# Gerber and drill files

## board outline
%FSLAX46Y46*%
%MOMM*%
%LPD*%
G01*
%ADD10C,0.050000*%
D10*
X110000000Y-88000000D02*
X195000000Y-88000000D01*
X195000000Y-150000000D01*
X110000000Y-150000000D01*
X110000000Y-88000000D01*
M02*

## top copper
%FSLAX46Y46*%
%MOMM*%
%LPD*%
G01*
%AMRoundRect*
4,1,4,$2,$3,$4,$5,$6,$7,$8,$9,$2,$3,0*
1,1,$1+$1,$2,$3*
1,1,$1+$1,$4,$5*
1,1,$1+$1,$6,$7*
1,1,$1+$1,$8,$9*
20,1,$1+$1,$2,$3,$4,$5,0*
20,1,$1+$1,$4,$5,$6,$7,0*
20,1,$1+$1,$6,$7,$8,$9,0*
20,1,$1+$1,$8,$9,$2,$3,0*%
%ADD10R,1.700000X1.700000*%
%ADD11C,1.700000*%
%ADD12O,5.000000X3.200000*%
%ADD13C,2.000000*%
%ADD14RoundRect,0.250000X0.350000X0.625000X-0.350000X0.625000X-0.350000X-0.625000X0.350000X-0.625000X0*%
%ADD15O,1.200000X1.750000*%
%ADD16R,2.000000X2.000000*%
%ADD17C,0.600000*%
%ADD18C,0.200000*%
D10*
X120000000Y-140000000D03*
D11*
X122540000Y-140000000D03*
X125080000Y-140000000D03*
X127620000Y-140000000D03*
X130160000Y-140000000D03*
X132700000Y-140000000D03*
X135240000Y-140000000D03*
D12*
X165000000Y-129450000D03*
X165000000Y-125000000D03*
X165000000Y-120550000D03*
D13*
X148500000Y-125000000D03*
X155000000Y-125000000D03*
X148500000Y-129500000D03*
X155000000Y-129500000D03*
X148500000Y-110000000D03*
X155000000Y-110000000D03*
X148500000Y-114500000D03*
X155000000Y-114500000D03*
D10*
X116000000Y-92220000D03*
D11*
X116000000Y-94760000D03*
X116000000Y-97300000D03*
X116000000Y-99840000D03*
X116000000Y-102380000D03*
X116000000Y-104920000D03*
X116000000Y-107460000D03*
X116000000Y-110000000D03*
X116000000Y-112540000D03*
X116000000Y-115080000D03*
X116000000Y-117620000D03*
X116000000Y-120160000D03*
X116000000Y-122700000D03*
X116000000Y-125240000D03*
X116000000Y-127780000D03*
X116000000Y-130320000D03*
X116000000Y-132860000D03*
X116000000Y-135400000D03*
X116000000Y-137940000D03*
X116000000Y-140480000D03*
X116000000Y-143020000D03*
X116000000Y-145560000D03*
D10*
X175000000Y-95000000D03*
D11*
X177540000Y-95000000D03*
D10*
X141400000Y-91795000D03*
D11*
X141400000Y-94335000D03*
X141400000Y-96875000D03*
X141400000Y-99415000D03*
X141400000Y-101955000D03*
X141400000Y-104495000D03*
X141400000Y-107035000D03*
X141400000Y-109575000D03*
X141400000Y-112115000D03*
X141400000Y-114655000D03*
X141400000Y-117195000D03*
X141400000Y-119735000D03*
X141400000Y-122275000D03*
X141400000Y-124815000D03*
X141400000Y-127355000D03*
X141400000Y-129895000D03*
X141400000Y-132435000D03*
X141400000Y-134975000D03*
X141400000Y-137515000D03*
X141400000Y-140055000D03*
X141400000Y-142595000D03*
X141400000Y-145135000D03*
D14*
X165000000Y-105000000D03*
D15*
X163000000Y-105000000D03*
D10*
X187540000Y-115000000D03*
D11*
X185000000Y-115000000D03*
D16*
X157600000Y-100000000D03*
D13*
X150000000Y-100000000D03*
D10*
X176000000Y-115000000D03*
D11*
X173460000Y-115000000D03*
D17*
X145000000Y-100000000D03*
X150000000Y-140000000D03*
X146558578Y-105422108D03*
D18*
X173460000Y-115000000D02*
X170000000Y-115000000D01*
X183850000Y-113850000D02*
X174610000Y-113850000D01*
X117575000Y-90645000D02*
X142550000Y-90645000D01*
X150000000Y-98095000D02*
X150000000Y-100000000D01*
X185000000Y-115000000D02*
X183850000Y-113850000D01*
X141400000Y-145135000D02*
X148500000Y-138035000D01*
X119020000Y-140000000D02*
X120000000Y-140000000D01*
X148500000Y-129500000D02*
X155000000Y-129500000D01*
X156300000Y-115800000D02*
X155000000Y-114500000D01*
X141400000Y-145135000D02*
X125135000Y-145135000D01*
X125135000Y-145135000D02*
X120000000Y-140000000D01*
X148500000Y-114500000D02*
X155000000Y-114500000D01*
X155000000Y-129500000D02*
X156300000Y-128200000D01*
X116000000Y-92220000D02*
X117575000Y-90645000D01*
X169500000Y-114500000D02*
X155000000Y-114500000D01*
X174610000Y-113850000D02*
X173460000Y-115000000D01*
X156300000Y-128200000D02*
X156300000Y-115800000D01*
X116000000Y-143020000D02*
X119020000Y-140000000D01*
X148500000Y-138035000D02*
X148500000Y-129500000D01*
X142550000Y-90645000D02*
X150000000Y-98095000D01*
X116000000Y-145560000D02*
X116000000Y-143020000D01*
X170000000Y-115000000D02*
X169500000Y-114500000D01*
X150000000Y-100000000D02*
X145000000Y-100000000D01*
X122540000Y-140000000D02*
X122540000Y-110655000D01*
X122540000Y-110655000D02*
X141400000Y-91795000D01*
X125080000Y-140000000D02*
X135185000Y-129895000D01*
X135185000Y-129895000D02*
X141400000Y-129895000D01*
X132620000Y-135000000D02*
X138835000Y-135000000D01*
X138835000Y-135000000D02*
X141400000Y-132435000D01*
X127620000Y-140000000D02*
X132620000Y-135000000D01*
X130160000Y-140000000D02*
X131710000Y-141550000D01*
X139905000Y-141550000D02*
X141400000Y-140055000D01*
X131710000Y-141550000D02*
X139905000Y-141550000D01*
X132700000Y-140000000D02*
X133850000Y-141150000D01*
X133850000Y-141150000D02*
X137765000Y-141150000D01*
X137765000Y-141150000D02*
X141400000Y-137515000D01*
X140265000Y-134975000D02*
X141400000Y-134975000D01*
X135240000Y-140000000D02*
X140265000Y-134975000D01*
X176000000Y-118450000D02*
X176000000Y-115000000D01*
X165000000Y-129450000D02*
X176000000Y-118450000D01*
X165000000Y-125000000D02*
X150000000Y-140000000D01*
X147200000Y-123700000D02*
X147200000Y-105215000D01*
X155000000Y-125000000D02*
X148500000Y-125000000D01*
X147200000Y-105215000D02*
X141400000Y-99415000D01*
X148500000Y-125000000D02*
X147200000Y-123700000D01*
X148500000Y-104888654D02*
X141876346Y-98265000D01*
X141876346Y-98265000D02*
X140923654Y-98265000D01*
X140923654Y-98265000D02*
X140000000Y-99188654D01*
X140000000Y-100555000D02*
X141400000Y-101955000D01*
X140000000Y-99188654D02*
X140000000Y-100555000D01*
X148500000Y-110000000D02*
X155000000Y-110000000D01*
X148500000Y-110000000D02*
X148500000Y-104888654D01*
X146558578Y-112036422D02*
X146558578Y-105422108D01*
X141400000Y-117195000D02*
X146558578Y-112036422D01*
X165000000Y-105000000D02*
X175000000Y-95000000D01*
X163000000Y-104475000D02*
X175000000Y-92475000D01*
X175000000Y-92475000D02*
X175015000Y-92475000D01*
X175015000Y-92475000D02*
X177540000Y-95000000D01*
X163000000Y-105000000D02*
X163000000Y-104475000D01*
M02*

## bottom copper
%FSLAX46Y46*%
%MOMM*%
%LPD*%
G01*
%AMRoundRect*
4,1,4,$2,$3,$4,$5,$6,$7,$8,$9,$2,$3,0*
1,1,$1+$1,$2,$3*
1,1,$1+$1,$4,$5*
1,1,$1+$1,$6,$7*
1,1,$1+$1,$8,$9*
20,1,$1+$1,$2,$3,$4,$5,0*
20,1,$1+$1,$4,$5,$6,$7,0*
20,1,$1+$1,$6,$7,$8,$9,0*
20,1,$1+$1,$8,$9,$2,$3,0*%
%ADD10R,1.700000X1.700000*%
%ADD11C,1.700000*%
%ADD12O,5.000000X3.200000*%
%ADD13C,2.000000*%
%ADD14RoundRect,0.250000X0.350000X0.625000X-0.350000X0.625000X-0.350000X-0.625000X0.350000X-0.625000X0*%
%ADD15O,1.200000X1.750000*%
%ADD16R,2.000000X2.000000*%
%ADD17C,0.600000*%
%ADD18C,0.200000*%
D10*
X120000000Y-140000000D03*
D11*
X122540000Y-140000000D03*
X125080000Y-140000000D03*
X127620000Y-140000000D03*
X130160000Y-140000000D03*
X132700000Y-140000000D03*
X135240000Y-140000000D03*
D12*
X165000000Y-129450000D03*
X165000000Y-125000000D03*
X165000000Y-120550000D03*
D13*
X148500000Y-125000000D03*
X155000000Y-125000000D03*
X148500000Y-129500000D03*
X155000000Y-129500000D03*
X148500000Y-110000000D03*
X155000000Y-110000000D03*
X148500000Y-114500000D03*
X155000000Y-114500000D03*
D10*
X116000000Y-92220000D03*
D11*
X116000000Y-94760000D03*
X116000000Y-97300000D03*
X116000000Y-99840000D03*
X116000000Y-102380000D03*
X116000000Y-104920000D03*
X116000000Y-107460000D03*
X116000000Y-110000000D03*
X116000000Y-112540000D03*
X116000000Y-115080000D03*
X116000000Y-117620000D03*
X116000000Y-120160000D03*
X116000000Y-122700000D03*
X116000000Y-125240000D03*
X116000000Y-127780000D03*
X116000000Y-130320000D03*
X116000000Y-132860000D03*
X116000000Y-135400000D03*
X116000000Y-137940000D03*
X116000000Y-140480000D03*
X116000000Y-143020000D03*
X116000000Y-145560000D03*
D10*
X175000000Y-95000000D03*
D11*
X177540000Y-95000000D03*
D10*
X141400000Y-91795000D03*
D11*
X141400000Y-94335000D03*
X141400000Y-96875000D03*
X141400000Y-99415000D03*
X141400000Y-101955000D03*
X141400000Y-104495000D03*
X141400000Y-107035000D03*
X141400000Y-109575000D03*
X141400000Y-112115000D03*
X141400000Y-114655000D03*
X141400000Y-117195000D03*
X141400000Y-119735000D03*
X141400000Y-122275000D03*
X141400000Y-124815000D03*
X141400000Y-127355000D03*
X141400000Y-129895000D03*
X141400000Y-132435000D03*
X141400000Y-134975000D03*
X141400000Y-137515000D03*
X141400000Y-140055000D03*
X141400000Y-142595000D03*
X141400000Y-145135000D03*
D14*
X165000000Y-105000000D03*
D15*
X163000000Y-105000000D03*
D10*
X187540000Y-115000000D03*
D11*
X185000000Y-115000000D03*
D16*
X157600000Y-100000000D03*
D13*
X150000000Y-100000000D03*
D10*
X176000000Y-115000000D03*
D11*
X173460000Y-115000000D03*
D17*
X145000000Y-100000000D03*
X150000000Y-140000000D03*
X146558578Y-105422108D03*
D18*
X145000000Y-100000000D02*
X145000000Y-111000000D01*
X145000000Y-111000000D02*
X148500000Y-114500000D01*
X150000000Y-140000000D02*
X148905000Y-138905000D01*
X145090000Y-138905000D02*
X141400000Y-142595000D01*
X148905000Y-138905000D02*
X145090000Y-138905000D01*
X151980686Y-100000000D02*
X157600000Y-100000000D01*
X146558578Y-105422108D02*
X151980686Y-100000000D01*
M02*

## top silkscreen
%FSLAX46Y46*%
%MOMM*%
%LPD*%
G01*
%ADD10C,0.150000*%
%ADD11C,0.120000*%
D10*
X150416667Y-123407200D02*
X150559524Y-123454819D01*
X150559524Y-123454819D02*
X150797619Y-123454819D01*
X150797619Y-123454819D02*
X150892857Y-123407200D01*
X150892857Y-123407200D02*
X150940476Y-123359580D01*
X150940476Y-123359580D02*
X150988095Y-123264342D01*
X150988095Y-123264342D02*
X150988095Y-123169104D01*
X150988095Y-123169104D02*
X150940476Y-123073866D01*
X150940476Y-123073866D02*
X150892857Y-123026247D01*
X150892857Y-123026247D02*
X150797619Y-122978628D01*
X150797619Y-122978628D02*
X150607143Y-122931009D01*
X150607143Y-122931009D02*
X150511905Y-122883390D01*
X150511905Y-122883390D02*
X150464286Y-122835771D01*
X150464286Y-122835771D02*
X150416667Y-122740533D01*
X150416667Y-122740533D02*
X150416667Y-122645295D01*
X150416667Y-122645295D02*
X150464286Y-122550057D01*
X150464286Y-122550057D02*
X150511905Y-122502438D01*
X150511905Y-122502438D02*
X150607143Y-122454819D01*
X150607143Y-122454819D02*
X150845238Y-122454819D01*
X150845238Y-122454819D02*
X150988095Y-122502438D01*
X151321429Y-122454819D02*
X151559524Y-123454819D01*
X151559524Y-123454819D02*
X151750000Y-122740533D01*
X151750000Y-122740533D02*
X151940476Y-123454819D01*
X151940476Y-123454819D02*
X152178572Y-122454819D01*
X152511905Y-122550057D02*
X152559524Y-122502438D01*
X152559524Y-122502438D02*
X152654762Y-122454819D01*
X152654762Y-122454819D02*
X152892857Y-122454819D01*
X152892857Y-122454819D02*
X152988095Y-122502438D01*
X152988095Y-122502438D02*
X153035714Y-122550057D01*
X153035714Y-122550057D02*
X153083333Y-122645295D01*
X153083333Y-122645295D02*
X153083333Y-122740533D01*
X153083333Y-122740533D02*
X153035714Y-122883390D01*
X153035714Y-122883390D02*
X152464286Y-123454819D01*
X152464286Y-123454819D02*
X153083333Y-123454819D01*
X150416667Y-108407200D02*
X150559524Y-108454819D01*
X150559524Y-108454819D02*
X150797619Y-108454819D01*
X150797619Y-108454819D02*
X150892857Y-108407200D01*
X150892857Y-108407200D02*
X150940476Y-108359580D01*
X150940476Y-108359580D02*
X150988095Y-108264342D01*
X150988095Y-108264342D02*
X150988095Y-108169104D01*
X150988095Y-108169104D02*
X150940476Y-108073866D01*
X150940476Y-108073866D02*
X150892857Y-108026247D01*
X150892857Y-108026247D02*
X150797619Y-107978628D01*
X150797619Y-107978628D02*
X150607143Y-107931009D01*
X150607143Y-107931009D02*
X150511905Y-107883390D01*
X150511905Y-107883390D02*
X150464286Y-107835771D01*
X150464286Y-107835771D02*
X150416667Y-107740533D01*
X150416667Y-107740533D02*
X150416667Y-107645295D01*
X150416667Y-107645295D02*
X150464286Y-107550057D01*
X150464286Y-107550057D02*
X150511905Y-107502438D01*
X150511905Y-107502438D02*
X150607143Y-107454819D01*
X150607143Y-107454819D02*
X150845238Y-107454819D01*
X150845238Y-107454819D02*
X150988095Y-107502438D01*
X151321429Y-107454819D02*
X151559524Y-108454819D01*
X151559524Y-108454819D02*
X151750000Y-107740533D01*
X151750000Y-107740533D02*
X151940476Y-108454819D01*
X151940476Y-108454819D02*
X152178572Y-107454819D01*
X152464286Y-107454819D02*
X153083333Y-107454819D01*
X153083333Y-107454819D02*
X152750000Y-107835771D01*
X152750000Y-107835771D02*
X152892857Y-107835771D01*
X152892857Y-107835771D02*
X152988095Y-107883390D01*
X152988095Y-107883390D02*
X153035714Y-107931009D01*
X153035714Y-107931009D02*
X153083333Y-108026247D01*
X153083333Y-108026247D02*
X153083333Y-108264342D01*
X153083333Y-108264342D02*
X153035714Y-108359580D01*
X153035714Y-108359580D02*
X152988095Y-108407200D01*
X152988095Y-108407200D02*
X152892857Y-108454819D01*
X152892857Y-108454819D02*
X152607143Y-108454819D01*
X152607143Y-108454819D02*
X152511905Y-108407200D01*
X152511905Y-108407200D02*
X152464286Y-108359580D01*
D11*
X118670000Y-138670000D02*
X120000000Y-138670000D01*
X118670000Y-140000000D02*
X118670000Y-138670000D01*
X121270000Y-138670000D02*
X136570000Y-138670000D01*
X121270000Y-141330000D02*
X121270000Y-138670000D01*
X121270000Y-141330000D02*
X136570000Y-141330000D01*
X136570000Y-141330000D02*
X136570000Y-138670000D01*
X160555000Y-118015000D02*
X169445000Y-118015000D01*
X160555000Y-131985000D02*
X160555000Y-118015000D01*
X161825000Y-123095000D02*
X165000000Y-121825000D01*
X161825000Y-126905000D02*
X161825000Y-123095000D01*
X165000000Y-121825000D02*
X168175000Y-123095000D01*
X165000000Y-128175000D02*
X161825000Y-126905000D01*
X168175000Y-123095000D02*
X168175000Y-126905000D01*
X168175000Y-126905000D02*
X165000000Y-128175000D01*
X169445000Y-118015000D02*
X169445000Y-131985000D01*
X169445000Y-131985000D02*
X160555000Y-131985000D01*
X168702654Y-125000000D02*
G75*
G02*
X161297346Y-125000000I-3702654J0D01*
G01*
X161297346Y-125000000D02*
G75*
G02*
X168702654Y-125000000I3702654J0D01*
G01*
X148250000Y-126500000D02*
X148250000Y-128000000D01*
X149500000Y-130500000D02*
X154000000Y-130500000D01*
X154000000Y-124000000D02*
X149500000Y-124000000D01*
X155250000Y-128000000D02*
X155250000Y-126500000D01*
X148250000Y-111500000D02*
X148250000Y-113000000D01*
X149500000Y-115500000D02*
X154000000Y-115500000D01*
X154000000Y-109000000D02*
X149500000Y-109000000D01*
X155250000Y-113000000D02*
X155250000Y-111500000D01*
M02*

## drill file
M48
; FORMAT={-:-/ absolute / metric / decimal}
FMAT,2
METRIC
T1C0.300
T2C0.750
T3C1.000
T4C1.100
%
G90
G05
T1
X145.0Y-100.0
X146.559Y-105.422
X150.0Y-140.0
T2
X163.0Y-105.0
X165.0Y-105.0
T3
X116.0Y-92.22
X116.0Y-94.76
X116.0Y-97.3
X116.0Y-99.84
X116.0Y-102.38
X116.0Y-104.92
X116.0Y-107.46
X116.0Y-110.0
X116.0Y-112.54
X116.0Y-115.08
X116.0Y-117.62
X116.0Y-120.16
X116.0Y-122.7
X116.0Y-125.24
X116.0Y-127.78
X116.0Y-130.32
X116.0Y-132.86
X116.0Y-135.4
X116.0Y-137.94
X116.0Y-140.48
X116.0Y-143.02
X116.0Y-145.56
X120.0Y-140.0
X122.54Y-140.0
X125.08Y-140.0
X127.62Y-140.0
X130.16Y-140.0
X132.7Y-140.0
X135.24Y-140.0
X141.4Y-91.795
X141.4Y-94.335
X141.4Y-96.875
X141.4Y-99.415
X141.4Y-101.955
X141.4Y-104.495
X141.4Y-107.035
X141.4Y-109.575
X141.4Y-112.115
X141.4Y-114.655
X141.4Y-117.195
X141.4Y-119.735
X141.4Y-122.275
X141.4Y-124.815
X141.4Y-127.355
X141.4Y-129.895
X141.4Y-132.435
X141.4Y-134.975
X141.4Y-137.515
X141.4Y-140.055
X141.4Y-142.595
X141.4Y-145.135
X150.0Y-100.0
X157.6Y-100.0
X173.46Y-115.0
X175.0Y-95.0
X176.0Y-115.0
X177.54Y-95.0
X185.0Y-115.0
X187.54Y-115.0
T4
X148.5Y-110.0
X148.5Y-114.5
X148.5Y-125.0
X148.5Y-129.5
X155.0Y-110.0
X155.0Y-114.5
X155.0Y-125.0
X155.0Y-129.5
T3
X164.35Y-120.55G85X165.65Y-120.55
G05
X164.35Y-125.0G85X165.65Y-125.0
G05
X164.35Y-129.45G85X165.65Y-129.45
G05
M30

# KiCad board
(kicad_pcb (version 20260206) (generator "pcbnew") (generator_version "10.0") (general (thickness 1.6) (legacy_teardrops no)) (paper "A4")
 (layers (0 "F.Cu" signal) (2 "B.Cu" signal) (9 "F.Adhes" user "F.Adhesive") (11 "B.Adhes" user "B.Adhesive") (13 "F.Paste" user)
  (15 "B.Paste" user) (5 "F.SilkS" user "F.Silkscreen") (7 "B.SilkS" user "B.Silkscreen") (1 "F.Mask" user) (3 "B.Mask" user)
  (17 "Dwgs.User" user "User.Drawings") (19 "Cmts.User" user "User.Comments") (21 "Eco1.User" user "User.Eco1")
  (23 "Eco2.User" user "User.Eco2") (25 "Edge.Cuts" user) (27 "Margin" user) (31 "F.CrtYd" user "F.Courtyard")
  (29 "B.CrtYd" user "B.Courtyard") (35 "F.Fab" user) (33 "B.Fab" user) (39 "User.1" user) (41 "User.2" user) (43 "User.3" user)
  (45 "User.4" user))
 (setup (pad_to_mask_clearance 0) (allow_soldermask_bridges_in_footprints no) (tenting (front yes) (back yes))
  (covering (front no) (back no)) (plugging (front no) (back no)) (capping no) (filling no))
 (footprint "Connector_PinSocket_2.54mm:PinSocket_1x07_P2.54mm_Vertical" (layer "F.Cu") (at 120 140 90)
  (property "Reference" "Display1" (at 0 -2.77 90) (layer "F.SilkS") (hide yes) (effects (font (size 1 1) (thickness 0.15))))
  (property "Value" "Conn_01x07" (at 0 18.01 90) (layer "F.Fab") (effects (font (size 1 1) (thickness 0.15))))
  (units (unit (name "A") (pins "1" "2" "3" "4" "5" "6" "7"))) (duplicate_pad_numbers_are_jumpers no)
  (fp_line (start 1.33 -1.33) (end 1.33 0) (stroke (width 0.12) (type solid)) (layer "F.SilkS"))
  (fp_line (start 0 -1.33) (end 1.33 -1.33) (stroke (width 0.12) (type solid)) (layer "F.SilkS"))
  (fp_line (start 1.33 1.27) (end 1.33 16.57) (stroke (width 0.12) (type solid)) (layer "F.SilkS"))
  (fp_line (start -1.33 1.27) (end 1.33 1.27) (stroke (width 0.12) (type solid)) (layer "F.SilkS"))
  (fp_line (start -1.33 1.27) (end -1.33 16.57) (stroke (width 0.12) (type solid)) (layer "F.SilkS"))
  (fp_line (start -1.33 16.57) (end 1.33 16.57) (stroke (width 0.12) (type solid)) (layer "F.SilkS"))
  (pad "1" thru_hole rect (at 0 0 90) (size 1.7 1.7) (drill 1) (layers "*.Cu" "*.Mask") (remove_unused_layers no) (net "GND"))
  (pad "2" thru_hole circle (at 0 2.54 90) (size 1.7 1.7) (drill 1) (layers "*.Cu" "*.Mask") (remove_unused_layers no) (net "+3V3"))
  (pad "3" thru_hole circle (at 0 5.08 90) (size 1.7 1.7) (drill 1) (layers "*.Cu" "*.Mask") (remove_unused_layers no) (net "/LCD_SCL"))
  (pad "4" thru_hole circle (at 0 7.62 90) (size 1.7 1.7) (drill 1) (layers "*.Cu" "*.Mask") (remove_unused_layers no) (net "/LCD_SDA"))
  (pad "5" thru_hole circle (at 0 10.16 90) (size 1.7 1.7) (drill 1) (layers "*.Cu" "*.Mask") (remove_unused_layers no) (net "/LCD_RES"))
  (pad "6" thru_hole circle (at 0 12.7 90) (size 1.7 1.7) (drill 1) (layers "*.Cu" "*.Mask") (remove_unused_layers no) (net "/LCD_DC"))
  (pad "7" thru_hole circle (at 0 15.24 90) (size 1.7 1.7) (drill 1) (layers "*.Cu" "*.Mask") (remove_unused_layers no) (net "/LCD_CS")))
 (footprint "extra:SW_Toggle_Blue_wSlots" (layer "F.Cu") (at 165 125 90)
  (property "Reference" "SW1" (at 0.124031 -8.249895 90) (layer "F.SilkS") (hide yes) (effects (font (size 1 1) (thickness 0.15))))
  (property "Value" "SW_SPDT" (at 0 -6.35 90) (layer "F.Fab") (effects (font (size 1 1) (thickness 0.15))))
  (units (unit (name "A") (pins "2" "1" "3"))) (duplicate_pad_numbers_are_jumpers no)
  (fp_line (start 6.985 -4.445) (end 6.985 4.445) (stroke (width 0.12) (type solid)) (layer "F.SilkS"))
  (fp_line (start -6.985 -4.445) (end 6.985 -4.445) (stroke (width 0.12) (type solid)) (layer "F.SilkS"))
  (fp_line (start 1.905 -3.175) (end 3.175 0) (stroke (width 0.12) (type solid)) (layer "F.SilkS"))
  (fp_line (start -1.905 -3.175) (end 1.905 -3.175) (stroke (width 0.12) (type solid)) (layer "F.SilkS"))
  (fp_line (start 3.175 0) (end 1.905 3.175) (stroke (width 0.12) (type solid)) (layer "F.SilkS"))
  (fp_line (start -3.175 0) (end -1.905 -3.175) (stroke (width 0.12) (type solid)) (layer "F.SilkS"))
  (fp_line (start 1.905 3.175) (end -1.905 3.175) (stroke (width 0.12) (type solid)) (layer "F.SilkS"))
  (fp_line (start -1.905 3.175) (end -3.175 0) (stroke (width 0.12) (type solid)) (layer "F.SilkS"))
  (fp_line (start 6.985 4.445) (end -6.985 4.445) (stroke (width 0.12) (type solid)) (layer "F.SilkS"))
  (fp_line (start -6.985 4.445) (end -6.985 -4.445) (stroke (width 0.12) (type solid)) (layer "F.SilkS"))
  (fp_circle (center 0 0) (end 1.905 3.175) (stroke (width 0.12) (type solid)) (fill no) (layer "F.SilkS"))
  (pad "1" thru_hole oval (at -4.45 0 90) (size 3.2 5) (drill oval 1 2.3) (layers "*.Cu") (remove_unused_layers no) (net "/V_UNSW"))
  (pad "2" thru_hole oval (at 0 0 90) (size 3.2 5) (drill oval 1 2.3) (layers "*.Cu") (remove_unused_layers no) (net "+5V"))
  (pad "3" thru_hole oval (at 4.45 0 90) (size 3.2 5) (drill oval 1 2.3) (layers "*.Cu") (remove_unused_layers no)
   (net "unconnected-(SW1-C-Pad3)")))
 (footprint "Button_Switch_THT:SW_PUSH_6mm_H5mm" (layer "F.Cu") (at 148.5 125)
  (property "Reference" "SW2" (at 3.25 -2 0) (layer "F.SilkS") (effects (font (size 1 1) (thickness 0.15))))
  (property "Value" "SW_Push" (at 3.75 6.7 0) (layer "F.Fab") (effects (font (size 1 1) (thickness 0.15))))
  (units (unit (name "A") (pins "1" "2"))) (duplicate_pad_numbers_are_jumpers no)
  (fp_line (start -0.25 1.5) (end -0.25 3) (stroke (width 0.12) (type solid)) (layer "F.SilkS"))
  (fp_line (start 1 5.5) (end 5.5 5.5) (stroke (width 0.12) (type solid)) (layer "F.SilkS"))
  (fp_line (start 5.5 -1) (end 1 -1) (stroke (width 0.12) (type solid)) (layer "F.SilkS"))
  (fp_line (start 6.75 3) (end 6.75 1.5) (stroke (width 0.12) (type solid)) (layer "F.SilkS"))
  (pad "1" thru_hole circle (at 0 0 90) (size 2 2) (drill 1.1) (layers "*.Cu" "*.Mask") (remove_unused_layers no) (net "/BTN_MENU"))
  (pad "1" thru_hole circle (at 6.5 0 90) (size 2 2) (drill 1.1) (layers "*.Cu" "*.Mask") (remove_unused_layers no) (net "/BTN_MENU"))
  (pad "2" thru_hole circle (at 0 4.5 90) (size 2 2) (drill 1.1) (layers "*.Cu" "*.Mask") (remove_unused_layers no) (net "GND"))
  (pad "2" thru_hole circle (at 6.5 4.5 90) (size 2 2) (drill 1.1) (layers "*.Cu" "*.Mask") (remove_unused_layers no) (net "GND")))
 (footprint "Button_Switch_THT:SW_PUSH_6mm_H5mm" (layer "F.Cu") (at 148.5 110)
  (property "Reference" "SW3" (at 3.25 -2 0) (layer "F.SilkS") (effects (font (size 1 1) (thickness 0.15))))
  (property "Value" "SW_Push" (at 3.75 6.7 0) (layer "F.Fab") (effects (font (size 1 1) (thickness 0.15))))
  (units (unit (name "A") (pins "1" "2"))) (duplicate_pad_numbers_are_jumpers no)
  (fp_line (start -0.25 1.5) (end -0.25 3) (stroke (width 0.12) (type solid)) (layer "F.SilkS"))
  (fp_line (start 1 5.5) (end 5.5 5.5) (stroke (width 0.12) (type solid)) (layer "F.SilkS"))
  (fp_line (start 5.5 -1) (end 1 -1) (stroke (width 0.12) (type solid)) (layer "F.SilkS"))
  (fp_line (start 6.75 3) (end 6.75 1.5) (stroke (width 0.12) (type solid)) (layer "F.SilkS"))
  (pad "1" thru_hole circle (at 0 0 90) (size 2 2) (drill 1.1) (layers "*.Cu" "*.Mask") (remove_unused_layers no) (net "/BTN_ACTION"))
  (pad "1" thru_hole circle (at 6.5 0 90) (size 2 2) (drill 1.1) (layers "*.Cu" "*.Mask") (remove_unused_layers no) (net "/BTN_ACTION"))
  (pad "2" thru_hole circle (at 0 4.5 90) (size 2 2) (drill 1.1) (layers "*.Cu" "*.Mask") (remove_unused_layers no) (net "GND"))
  (pad "2" thru_hole circle (at 6.5 4.5 90) (size 2 2) (drill 1.1) (layers "*.Cu" "*.Mask") (remove_unused_layers no) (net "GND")))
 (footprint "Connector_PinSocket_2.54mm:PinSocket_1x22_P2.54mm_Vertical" (layer "B.Cu") (at 116 92.22 180)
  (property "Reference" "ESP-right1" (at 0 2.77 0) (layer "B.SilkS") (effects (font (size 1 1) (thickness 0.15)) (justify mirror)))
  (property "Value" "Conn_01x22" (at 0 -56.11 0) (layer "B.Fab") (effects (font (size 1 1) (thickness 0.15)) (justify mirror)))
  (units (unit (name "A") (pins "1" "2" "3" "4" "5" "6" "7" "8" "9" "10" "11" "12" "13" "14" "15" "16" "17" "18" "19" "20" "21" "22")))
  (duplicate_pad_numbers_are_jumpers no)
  (pad "1" thru_hole rect (at 0 0 180) (size 1.7 1.7) (drill 1) (layers "*.Cu" "*.Mask") (remove_unused_layers no) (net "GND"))
  (pad "2" thru_hole circle (at 0 -2.54 180) (size 1.7 1.7) (drill 1) (layers "*.Cu" "*.Mask") (remove_unused_layers no)
   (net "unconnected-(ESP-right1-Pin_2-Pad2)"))
  (pad "3" thru_hole circle (at 0 -5.08 180) (size 1.7 1.7) (drill 1) (layers "*.Cu" "*.Mask") (remove_unused_layers no)
   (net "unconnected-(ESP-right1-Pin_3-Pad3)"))
  (pad "4" thru_hole circle (at 0 -7.62 180) (size 1.7 1.7) (drill 1) (layers "*.Cu" "*.Mask") (remove_unused_layers no)
   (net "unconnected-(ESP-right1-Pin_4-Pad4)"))
  (pad "5" thru_hole circle (at 0 -10.16 180) (size 1.7 1.7) (drill 1) (layers "*.Cu" "*.Mask") (remove_unused_layers no)
   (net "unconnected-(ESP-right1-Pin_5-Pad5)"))
  (pad "6" thru_hole circle (at 0 -12.7 180) (size 1.7 1.7) (drill 1) (layers "*.Cu" "*.Mask") (remove_unused_layers no)
   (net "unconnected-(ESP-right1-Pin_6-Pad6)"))
  (pad "7" thru_hole circle (at 0 -15.24 180) (size 1.7 1.7) (drill 1) (layers "*.Cu" "*.Mask") (remove_unused_layers no)
   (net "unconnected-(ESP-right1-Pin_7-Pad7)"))
  (pad "8" thru_hole circle (at 0 -17.78 180) (size 1.7 1.7) (drill 1) (layers "*.Cu" "*.Mask") (remove_unused_layers no)
   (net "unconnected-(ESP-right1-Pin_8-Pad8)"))
  (pad "9" thru_hole circle (at 0 -20.32 180) (size 1.7 1.7) (drill 1) (layers "*.Cu" "*.Mask") (remove_unused_layers no)
   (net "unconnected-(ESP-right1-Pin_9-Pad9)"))
  (pad "10" thru_hole circle (at 0 -22.86 180) (size 1.7 1.7) (drill 1) (layers "*.Cu" "*.Mask") (remove_unused_layers no)
   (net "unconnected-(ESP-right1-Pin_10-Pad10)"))
  (pad "11" thru_hole circle (at 0 -25.4 180) (size 1.7 1.7) (drill 1) (layers "*.Cu" "*.Mask") (remove_unused_layers no)
   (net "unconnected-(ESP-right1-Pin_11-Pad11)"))
  (pad "12" thru_hole circle (at 0 -27.94 180) (size 1.7 1.7) (drill 1) (layers "*.Cu" "*.Mask") (remove_unused_layers no)
   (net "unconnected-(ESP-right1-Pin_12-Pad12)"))
  (pad "13" thru_hole circle (at 0 -30.48 180) (size 1.7 1.7) (drill 1) (layers "*.Cu" "*.Mask") (remove_unused_layers no)
   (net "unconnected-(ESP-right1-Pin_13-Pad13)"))
  (pad "14" thru_hole circle (at 0 -33.02 180) (size 1.7 1.7) (drill 1) (layers "*.Cu" "*.Mask") (remove_unused_layers no)
   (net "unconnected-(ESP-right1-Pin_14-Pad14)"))
  (pad "15" thru_hole circle (at 0 -35.56 180) (size 1.7 1.7) (drill 1) (layers "*.Cu" "*.Mask") (remove_unused_layers no)
   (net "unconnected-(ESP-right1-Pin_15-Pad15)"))
  (pad "16" thru_hole circle (at 0 -38.1 180) (size 1.7 1.7) (drill 1) (layers "*.Cu" "*.Mask") (remove_unused_layers no)
   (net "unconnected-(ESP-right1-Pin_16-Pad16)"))
  (pad "17" thru_hole circle (at 0 -40.64 180) (size 1.7 1.7) (drill 1) (layers "*.Cu" "*.Mask") (remove_unused_layers no)
   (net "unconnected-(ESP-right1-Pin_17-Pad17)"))
  (pad "18" thru_hole circle (at 0 -43.18 180) (size 1.7 1.7) (drill 1) (layers "*.Cu" "*.Mask") (remove_unused_layers no)
   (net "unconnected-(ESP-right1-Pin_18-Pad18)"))
  (pad "19" thru_hole circle (at 0 -45.72 180) (size 1.7 1.7) (drill 1) (layers "*.Cu" "*.Mask") (remove_unused_layers no)
   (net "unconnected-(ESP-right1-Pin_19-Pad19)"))
  (pad "20" thru_hole circle (at 0 -48.26 180) (size 1.7 1.7) (drill 1) (layers "*.Cu" "*.Mask") (remove_unused_layers no)
   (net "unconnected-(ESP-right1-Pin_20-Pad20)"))
  (pad "21" thru_hole circle (at 0 -50.8 180) (size 1.7 1.7) (drill 1) (layers "*.Cu" "*.Mask") (remove_unused_layers no) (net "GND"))
  (pad "22" thru_hole circle (at 0 -53.34 180) (size 1.7 1.7) (drill 1) (layers "*.Cu" "*.Mask") (remove_unused_layers no) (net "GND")))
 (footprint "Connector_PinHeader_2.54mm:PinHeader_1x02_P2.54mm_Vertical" (layer "B.Cu") (at 175 95 -90)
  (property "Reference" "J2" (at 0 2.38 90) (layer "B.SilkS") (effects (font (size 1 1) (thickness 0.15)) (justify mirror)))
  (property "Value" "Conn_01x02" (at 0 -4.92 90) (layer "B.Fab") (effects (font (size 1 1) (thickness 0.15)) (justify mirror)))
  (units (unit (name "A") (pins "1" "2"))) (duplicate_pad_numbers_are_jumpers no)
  (pad "1" thru_hole rect (at 0 0 270) (size 1.7 1.7) (drill 1) (layers "*.Cu" "*.Mask") (remove_unused_layers no) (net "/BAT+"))
  (pad "2" thru_hole circle (at 0 -2.54 270) (size 1.7 1.7) (drill 1) (layers "*.Cu" "*.Mask") (remove_unused_layers no) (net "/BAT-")))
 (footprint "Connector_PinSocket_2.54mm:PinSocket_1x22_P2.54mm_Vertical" (layer "B.Cu") (at 141.4 91.795 180)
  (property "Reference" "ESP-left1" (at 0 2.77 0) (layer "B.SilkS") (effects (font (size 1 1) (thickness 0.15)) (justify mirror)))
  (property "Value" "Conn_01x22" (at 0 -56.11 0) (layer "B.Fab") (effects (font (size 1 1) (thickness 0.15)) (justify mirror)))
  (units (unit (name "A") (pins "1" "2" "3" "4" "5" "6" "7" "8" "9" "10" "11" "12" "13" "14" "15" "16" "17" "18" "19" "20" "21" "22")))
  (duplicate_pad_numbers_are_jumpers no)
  (pad "1" thru_hole rect (at 0 0 180) (size 1.7 1.7) (drill 1) (layers "*.Cu" "*.Mask") (remove_unused_layers no) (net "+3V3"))
  (pad "2" thru_hole circle (at 0 -2.54 180) (size 1.7 1.7) (drill 1) (layers "*.Cu" "*.Mask") (remove_unused_layers no)
   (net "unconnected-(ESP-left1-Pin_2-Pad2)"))
  (pad "3" thru_hole circle (at 0 -5.08 180) (size 1.7 1.7) (drill 1) (layers "*.Cu" "*.Mask") (remove_unused_layers no)
   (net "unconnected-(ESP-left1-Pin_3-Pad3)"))
  (pad "4" thru_hole circle (at 0 -7.62 180) (size 1.7 1.7) (drill 1) (layers "*.Cu" "*.Mask") (remove_unused_layers no) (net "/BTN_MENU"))
  (pad "5" thru_hole circle (at 0 -10.16 180) (size 1.7 1.7) (drill 1) (layers "*.Cu" "*.Mask") (remove_unused_layers no)
   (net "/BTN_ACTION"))
  (pad "6" thru_hole circle (at 0 -12.7 180) (size 1.7 1.7) (drill 1) (layers "*.Cu" "*.Mask") (remove_unused_layers no)
   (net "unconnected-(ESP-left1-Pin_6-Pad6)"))
  (pad "7" thru_hole circle (at 0 -15.24 180) (size 1.7 1.7) (drill 1) (layers "*.Cu" "*.Mask") (remove_unused_layers no)
   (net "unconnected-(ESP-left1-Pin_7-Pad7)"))
  (pad "8" thru_hole circle (at 0 -17.78 180) (size 1.7 1.7) (drill 1) (layers "*.Cu" "*.Mask") (remove_unused_layers no)
   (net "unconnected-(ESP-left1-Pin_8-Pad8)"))
  (pad "9" thru_hole circle (at 0 -20.32 180) (size 1.7 1.7) (drill 1) (layers "*.Cu" "*.Mask") (remove_unused_layers no)
   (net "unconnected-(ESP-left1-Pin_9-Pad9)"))
  (pad "10" thru_hole circle (at 0 -22.86 180) (size 1.7 1.7) (drill 1) (layers "*.Cu" "*.Mask") (remove_unused_layers no)
   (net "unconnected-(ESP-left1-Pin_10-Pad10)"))
  (pad "11" thru_hole circle (at 0 -25.4 180) (size 1.7 1.7) (drill 1) (layers "*.Cu" "*.Mask") (remove_unused_layers no) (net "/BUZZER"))
  (pad "12" thru_hole circle (at 0 -27.94 180) (size 1.7 1.7) (drill 1) (layers "*.Cu" "*.Mask") (remove_unused_layers no)
   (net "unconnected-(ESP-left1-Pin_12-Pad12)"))
  (pad "13" thru_hole circle (at 0 -30.48 180) (size 1.7 1.7) (drill 1) (layers "*.Cu" "*.Mask") (remove_unused_layers no)
   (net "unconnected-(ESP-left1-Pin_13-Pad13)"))
  (pad "14" thru_hole circle (at 0 -33.02 180) (size 1.7 1.7) (drill 1) (layers "*.Cu" "*.Mask") (remove_unused_layers no)
   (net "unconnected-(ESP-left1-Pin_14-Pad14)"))
  (pad "15" thru_hole circle (at 0 -35.56 180) (size 1.7 1.7) (drill 1) (layers "*.Cu" "*.Mask") (remove_unused_layers no)
   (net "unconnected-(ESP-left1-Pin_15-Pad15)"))
  (pad "16" thru_hole circle (at 0 -38.1 180) (size 1.7 1.7) (drill 1) (layers "*.Cu" "*.Mask") (remove_unused_layers no) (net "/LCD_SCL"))
  (pad "17" thru_hole circle (at 0 -40.64 180) (size 1.7 1.7) (drill 1) (layers "*.Cu" "*.Mask") (remove_unused_layers no) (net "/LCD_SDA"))
  (pad "18" thru_hole circle (at 0 -43.18 180) (size 1.7 1.7) (drill 1) (layers "*.Cu" "*.Mask") (remove_unused_layers no) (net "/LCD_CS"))
  (pad "19" thru_hole circle (at 0 -45.72 180) (size 1.7 1.7) (drill 1) (layers "*.Cu" "*.Mask") (remove_unused_layers no) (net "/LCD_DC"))
  (pad "20" thru_hole circle (at 0 -48.26 180) (size 1.7 1.7) (drill 1) (layers "*.Cu" "*.Mask") (remove_unused_layers no) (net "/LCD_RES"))
  (pad "21" thru_hole circle (at 0 -50.8 180) (size 1.7 1.7) (drill 1) (layers "*.Cu" "*.Mask") (remove_unused_layers no) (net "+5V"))
  (pad "22" thru_hole circle (at 0 -53.34 180) (size 1.7 1.7) (drill 1) (layers "*.Cu" "*.Mask") (remove_unused_layers no) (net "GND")))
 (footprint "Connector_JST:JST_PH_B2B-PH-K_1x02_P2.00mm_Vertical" (layer "B.Cu") (at 165 105 180)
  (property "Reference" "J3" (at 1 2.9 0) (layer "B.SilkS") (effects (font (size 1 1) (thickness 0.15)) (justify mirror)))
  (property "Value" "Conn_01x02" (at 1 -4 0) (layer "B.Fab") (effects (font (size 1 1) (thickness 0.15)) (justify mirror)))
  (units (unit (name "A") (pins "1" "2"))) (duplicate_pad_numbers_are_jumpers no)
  (pad "1" thru_hole roundrect (at 0 0 180) (size 1.2 1.75) (drill 0.75) (layers "*.Cu" "*.Mask") (remove_unused_layers no)
   (roundrect_rratio 0.208333) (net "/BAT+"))
  (pad "2" thru_hole oval (at 2 0 180) (size 1.2 1.75) (drill 0.75) (layers "*.Cu" "*.Mask") (remove_unused_layers no) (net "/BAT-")))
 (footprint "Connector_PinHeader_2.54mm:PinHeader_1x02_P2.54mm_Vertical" (layer "B.Cu") (at 187.54 115 90)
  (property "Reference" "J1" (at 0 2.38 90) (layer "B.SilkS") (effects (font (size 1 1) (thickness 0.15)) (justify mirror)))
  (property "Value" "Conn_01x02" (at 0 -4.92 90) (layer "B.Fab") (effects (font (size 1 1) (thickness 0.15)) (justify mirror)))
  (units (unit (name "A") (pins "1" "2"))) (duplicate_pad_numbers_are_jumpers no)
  (pad "1" thru_hole rect (at 0 0 90) (size 1.7 1.7) (drill 1) (layers "*.Cu" "*.Mask") (remove_unused_layers no)
   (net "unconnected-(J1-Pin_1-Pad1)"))
  (pad "2" thru_hole circle (at 0 -2.54 90) (size 1.7 1.7) (drill 1) (layers "*.Cu" "*.Mask") (remove_unused_layers no) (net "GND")))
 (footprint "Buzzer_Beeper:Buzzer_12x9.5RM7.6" (layer "B.Cu") (at 157.6 100 180)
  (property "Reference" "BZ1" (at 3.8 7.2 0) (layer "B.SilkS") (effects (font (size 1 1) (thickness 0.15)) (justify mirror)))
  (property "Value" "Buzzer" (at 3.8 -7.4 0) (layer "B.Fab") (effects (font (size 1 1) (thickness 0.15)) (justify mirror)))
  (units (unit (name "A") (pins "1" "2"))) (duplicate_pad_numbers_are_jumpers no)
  (pad "1" thru_hole rect (at 0 0 180) (size 2 2) (drill 1) (layers "*.Cu" "*.Mask") (remove_unused_layers no) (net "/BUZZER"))
  (pad "2" thru_hole circle (at 7.6 0 180) (size 2 2) (drill 1) (layers "*.Cu" "*.Mask") (remove_unused_layers no) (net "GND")))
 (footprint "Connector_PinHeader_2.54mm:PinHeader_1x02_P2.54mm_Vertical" (layer "B.Cu") (at 176 115 90)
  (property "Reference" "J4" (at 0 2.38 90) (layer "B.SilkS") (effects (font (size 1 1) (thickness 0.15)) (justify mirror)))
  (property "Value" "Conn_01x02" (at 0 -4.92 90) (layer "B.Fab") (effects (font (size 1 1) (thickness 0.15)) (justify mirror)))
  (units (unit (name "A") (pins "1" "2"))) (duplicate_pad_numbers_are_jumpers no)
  (pad "1" thru_hole rect (at 0 0 90) (size 1.7 1.7) (drill 1) (layers "*.Cu" "*.Mask") (remove_unused_layers no) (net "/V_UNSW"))
  (pad "2" thru_hole circle (at 0 -2.54 90) (size 1.7 1.7) (drill 1) (layers "*.Cu" "*.Mask") (remove_unused_layers no) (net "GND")))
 (gr_rect (start 110 88) (end 195 150) (stroke (width 0.05) (type default)) (fill no) (layer "Edge.Cuts"))
 (segment (start 173.46 115) (end 170 115) (width 0.2) (layer "F.Cu") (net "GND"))
 (segment (start 183.85 113.85) (end 174.61 113.85) (width 0.2) (layer "F.Cu") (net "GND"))
 (segment (start 117.575 90.645) (end 142.55 90.645) (width 0.2) (layer "F.Cu") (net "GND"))
 (segment (start 150 98.095) (end 150 100) (width 0.2) (layer "F.Cu") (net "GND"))
 (segment (start 185 115) (end 183.85 113.85) (width 0.2) (layer "F.Cu") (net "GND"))
 (segment (start 141.4 145.135) (end 148.5 138.035) (width 0.2) (layer "F.Cu") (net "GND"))
 (segment (start 119.02 140) (end 120 140) (width 0.2) (layer "F.Cu") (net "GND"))
 (segment (start 148.5 129.5) (end 155 129.5) (width 0.2) (layer "F.Cu") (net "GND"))
 (segment (start 156.3 115.8) (end 155 114.5) (width 0.2) (layer "F.Cu") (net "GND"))
 (segment (start 141.4 145.135) (end 125.135 145.135) (width 0.2) (layer "F.Cu") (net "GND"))
 (segment (start 125.135 145.135) (end 120 140) (width 0.2) (layer "F.Cu") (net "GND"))
 (segment (start 148.5 114.5) (end 155 114.5) (width 0.2) (layer "F.Cu") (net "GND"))
 (segment (start 155 129.5) (end 156.3 128.2) (width 0.2) (layer "F.Cu") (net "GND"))
 (segment (start 116 92.22) (end 117.575 90.645) (width 0.2) (layer "F.Cu") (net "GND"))
 (segment (start 169.5 114.5) (end 155 114.5) (width 0.2) (layer "F.Cu") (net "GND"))
 (segment (start 174.61 113.85) (end 173.46 115) (width 0.2) (layer "F.Cu") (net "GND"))
 (segment (start 156.3 128.2) (end 156.3 115.8) (width 0.2) (layer "F.Cu") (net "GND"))
 (segment (start 116 143.02) (end 119.02 140) (width 0.2) (layer "F.Cu") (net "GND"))
 (segment (start 148.5 138.035) (end 148.5 129.5) (width 0.2) (layer "F.Cu") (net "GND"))
 (segment (start 142.55 90.645) (end 150 98.095) (width 0.2) (layer "F.Cu") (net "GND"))
 (segment (start 116 145.56) (end 116 143.02) (width 0.2) (layer "F.Cu") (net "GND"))
 (segment (start 170 115) (end 169.5 114.5) (width 0.2) (layer "F.Cu") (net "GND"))
 (segment (start 150 100) (end 145 100) (width 0.2) (layer "F.Cu") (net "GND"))
 (via (at 145 100) (size 0.6) (drill 0.3) (layers "F.Cu" "B.Cu") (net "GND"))
 (segment (start 145 100) (end 145 111) (width 0.2) (layer "B.Cu") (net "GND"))
 (segment (start 145 111) (end 148.5 114.5) (width 0.2) (layer "B.Cu") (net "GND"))
 (segment (start 122.54 140) (end 122.54 110.655) (width 0.2) (layer "F.Cu") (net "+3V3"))
 (segment (start 122.54 110.655) (end 141.4 91.795) (width 0.2) (layer "F.Cu") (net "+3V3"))
 (segment (start 125.08 140) (end 135.185 129.895) (width 0.2) (layer "F.Cu") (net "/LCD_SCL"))
 (segment (start 135.185 129.895) (end 141.4 129.895) (width 0.2) (layer "F.Cu") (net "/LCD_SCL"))
 (segment (start 132.62 135) (end 138.835 135) (width 0.2) (layer "F.Cu") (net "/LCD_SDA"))
 (segment (start 138.835 135) (end 141.4 132.435) (width 0.2) (layer "F.Cu") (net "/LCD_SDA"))
 (segment (start 127.62 140) (end 132.62 135) (width 0.2) (layer "F.Cu") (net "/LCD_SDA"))
 (segment (start 130.16 140) (end 131.71 141.55) (width 0.2) (layer "F.Cu") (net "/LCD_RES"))
 (segment (start 139.905 141.55) (end 141.4 140.055) (width 0.2) (layer "F.Cu") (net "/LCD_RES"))
 (segment (start 131.71 141.55) (end 139.905 141.55) (width 0.2) (layer "F.Cu") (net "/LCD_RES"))
 (segment (start 132.7 140) (end 133.85 141.15) (width 0.2) (layer "F.Cu") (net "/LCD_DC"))
 (segment (start 133.85 141.15) (end 137.765 141.15) (width 0.2) (layer "F.Cu") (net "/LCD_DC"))
 (segment (start 137.765 141.15) (end 141.4 137.515) (width 0.2) (layer "F.Cu") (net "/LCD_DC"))
 (segment (start 140.265 134.975) (end 141.4 134.975) (width 0.2) (layer "F.Cu") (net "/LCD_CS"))
 (segment (start 135.24 140) (end 140.265 134.975) (width 0.2) (layer "F.Cu") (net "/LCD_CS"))
 (segment (start 176 118.45) (end 176 115) (width 0.2) (layer "F.Cu") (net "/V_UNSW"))
 (segment (start 165 129.45) (end 176 118.45) (width 0.2) (layer "F.Cu") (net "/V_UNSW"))
 (segment (start 165 125) (end 150 140) (width 0.2) (layer "F.Cu") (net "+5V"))
 (via (at 150 140) (size 0.6) (drill 0.3) (layers "F.Cu" "B.Cu") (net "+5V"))
 (segment (start 150 140) (end 148.905 138.905) (width 0.2) (layer "B.Cu") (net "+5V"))
 (segment (start 145.09 138.905) (end 141.4 142.595) (width 0.2) (layer "B.Cu") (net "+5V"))
 (segment (start 148.905 138.905) (end 145.09 138.905) (width 0.2) (layer "B.Cu") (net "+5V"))
 (segment (start 147.2 123.7) (end 147.2 105.215) (width 0.2) (layer "F.Cu") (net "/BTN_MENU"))
 (segment (start 155 125) (end 148.5 125) (width 0.2) (layer "F.Cu") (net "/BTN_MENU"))
 (segment (start 147.2 105.215) (end 141.4 99.415) (width 0.2) (layer "F.Cu") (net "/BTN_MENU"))
 (segment (start 148.5 125) (end 147.2 123.7) (width 0.2) (layer "F.Cu") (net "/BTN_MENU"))
 (segment (start 148.5 104.888654) (end 141.876346 98.265) (width 0.2) (layer "F.Cu") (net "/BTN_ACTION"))
 (segment (start 141.876346 98.265) (end 140.923654 98.265) (width 0.2) (layer "F.Cu") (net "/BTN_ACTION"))
 (segment (start 140.923654 98.265) (end 140 99.188654) (width 0.2) (layer "F.Cu") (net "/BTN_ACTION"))
 (segment (start 140 100.555) (end 141.4 101.955) (width 0.2) (layer "F.Cu") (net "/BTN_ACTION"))
 (segment (start 140 99.188654) (end 140 100.555) (width 0.2) (layer "F.Cu") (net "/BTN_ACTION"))
 (segment (start 148.5 110) (end 155 110) (width 0.2) (layer "F.Cu") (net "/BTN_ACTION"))
 (segment (start 148.5 110) (end 148.5 104.888654) (width 0.2) (layer "F.Cu") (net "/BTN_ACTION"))
 (segment (start 146.558578 112.036422) (end 146.558578 105.422108) (width 0.2) (layer "F.Cu") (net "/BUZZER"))
 (segment (start 141.4 117.195) (end 146.558578 112.036422) (width 0.2) (layer "F.Cu") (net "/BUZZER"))
 (via (at 146.558578 105.422108) (size 0.6) (drill 0.3) (layers "F.Cu" "B.Cu") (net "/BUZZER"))
 (segment (start 151.980686 100) (end 157.6 100) (width 0.2) (layer "B.Cu") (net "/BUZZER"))
 (segment (start 146.558578 105.422108) (end 151.980686 100) (width 0.2) (layer "B.Cu") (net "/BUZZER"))
 (segment (start 165 105) (end 175 95) (width 0.2) (layer "F.Cu") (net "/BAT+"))
 (segment (start 163 104.475) (end 175 92.475) (width 0.2) (layer "F.Cu") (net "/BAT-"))
 (segment (start 175 92.475) (end 175.015 92.475) (width 0.2) (layer "F.Cu") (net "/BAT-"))
 (segment (start 175.015 92.475) (end 177.54 95) (width 0.2) (layer "F.Cu") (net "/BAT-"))
 (segment (start 163 105) (end 163 104.475) (width 0.2) (layer "F.Cu") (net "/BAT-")))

